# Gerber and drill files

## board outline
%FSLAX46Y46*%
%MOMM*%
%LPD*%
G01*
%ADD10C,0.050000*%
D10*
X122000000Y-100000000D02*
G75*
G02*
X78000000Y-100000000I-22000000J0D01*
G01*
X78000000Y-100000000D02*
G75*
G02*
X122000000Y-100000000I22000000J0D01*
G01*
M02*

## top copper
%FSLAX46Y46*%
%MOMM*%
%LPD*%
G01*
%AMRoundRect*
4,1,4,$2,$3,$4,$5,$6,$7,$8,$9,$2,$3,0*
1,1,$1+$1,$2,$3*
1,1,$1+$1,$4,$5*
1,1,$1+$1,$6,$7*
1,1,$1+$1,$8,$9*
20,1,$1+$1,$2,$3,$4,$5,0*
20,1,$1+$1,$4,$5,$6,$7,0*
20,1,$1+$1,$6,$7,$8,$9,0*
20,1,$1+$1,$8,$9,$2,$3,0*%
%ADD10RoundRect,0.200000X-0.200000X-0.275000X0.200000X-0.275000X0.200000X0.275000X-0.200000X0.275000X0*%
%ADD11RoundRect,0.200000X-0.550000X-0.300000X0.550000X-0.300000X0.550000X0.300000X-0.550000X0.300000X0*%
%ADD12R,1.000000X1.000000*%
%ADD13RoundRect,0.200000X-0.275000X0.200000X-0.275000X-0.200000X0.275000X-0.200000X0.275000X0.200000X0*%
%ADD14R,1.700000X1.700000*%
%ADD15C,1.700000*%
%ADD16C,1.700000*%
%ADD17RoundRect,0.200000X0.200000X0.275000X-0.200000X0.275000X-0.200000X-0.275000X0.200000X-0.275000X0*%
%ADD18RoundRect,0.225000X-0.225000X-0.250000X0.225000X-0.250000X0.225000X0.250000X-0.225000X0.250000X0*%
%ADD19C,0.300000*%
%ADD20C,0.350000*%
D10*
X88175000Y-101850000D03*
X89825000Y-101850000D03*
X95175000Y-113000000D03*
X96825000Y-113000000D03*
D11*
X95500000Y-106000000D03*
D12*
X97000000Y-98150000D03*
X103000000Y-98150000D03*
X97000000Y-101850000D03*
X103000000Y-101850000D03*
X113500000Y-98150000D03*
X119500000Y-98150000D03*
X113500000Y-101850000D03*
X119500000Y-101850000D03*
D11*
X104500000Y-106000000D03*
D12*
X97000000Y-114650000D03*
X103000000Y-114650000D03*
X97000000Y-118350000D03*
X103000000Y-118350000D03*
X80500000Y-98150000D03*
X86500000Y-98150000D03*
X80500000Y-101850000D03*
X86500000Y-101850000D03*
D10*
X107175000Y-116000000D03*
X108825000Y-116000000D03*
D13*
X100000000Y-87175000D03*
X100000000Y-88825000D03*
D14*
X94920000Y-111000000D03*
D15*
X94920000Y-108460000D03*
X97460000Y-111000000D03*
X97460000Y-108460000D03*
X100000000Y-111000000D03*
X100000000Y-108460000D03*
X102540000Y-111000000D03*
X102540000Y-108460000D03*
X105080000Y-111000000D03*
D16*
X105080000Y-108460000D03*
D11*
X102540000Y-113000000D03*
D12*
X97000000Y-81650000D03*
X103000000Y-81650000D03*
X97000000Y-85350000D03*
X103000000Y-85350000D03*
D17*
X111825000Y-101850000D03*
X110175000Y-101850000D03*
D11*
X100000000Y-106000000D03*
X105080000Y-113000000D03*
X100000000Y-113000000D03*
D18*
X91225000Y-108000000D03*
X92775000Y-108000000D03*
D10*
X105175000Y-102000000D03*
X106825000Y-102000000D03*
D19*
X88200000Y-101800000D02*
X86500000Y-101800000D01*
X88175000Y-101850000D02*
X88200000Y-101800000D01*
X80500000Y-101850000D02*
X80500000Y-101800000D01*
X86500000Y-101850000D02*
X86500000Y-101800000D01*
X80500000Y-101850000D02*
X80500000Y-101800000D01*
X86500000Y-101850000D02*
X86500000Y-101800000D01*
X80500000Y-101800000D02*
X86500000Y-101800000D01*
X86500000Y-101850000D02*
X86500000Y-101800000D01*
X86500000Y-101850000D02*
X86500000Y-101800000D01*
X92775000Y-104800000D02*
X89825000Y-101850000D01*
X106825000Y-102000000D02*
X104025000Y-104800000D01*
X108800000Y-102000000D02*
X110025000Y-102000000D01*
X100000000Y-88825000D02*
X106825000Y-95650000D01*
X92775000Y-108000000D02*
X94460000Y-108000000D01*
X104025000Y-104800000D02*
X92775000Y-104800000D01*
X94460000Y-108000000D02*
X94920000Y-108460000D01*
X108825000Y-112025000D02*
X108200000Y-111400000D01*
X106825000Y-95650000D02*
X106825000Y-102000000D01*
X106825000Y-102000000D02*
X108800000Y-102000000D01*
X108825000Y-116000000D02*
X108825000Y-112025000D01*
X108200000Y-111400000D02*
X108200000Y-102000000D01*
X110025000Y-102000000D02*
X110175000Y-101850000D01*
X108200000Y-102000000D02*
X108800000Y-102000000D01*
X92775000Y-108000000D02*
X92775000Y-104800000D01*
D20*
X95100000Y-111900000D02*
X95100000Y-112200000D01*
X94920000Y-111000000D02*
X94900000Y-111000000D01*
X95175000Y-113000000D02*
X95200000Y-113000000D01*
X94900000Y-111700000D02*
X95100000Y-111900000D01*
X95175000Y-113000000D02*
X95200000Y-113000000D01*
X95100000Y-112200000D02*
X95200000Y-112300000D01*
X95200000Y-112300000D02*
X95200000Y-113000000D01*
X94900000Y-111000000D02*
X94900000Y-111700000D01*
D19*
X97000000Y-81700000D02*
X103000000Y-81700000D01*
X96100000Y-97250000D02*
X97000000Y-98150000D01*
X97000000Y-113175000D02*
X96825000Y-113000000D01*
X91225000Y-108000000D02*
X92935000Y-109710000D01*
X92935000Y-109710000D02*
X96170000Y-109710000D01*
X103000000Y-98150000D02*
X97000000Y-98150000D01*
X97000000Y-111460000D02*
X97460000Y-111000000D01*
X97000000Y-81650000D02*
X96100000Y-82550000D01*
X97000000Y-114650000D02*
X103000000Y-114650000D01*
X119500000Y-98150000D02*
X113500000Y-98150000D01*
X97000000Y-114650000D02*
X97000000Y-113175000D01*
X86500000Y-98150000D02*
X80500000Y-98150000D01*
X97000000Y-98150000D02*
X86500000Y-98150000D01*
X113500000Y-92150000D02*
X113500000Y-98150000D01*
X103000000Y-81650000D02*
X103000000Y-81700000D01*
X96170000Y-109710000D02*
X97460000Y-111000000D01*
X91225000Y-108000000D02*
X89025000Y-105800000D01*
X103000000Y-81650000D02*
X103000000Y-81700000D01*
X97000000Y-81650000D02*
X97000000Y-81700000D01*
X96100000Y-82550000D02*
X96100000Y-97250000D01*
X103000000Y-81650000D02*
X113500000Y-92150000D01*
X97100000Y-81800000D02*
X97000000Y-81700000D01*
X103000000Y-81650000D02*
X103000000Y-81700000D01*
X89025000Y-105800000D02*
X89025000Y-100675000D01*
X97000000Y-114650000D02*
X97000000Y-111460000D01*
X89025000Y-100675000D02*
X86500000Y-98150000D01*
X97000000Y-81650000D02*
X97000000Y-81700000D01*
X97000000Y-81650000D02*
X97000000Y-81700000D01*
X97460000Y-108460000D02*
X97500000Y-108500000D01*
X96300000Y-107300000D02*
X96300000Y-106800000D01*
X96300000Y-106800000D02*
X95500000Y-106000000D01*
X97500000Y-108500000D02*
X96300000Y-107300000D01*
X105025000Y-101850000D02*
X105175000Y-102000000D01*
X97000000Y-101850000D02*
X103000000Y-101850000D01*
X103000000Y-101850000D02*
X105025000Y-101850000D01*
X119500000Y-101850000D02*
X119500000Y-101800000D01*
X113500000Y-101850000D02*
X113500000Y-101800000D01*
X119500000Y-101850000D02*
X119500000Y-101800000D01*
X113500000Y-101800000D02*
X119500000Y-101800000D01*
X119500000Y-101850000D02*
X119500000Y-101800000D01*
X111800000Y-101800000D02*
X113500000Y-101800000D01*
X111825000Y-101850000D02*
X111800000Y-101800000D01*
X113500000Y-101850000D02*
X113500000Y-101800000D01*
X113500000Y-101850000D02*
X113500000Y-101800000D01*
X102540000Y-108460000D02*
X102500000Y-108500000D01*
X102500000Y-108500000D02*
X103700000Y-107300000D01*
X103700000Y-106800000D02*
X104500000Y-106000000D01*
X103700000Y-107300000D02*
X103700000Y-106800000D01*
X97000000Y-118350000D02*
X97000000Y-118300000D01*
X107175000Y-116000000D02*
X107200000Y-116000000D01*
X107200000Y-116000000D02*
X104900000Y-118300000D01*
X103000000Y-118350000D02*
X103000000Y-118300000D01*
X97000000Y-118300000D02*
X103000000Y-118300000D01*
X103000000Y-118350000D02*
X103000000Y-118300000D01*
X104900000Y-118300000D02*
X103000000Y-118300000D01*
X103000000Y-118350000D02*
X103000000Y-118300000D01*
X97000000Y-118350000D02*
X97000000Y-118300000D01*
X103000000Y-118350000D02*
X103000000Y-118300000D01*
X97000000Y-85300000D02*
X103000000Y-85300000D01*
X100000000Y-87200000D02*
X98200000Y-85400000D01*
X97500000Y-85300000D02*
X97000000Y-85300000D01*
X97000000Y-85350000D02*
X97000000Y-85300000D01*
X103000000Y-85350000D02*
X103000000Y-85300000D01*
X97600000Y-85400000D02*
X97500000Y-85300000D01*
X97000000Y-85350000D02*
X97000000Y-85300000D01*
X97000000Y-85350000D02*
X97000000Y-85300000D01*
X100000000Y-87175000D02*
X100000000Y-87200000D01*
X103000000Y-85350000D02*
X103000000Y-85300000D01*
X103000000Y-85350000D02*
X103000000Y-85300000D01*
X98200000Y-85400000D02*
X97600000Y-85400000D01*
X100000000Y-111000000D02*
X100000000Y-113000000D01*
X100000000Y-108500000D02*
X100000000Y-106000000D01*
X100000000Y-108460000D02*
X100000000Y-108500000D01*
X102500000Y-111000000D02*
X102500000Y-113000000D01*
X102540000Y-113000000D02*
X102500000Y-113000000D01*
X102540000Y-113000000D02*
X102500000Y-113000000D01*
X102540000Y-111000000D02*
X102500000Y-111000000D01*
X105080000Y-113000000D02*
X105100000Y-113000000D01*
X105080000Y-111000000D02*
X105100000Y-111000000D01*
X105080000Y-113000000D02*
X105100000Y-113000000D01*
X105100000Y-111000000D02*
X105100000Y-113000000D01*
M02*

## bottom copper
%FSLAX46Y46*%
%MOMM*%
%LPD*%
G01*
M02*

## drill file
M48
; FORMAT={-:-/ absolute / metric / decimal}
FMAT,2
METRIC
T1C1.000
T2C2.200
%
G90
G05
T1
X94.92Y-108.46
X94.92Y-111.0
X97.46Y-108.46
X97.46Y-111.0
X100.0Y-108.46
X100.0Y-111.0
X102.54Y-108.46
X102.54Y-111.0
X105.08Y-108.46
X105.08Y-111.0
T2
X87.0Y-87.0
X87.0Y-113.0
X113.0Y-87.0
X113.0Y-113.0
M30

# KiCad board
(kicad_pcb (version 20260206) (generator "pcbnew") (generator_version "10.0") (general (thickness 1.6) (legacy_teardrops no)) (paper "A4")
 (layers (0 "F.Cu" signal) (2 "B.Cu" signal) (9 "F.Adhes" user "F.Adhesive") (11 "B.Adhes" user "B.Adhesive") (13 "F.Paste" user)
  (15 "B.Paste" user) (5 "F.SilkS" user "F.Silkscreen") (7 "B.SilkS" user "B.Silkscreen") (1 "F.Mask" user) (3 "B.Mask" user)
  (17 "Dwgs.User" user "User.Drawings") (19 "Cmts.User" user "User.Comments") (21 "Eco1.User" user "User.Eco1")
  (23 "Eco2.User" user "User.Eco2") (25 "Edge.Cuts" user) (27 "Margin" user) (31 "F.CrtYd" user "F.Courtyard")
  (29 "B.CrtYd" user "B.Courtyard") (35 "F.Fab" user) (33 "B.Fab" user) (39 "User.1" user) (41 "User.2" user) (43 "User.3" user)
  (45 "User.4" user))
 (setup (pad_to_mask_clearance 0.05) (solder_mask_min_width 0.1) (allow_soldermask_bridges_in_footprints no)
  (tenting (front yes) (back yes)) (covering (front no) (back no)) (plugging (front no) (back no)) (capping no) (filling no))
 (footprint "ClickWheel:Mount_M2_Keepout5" (layer "F.Cu") (at 87 113)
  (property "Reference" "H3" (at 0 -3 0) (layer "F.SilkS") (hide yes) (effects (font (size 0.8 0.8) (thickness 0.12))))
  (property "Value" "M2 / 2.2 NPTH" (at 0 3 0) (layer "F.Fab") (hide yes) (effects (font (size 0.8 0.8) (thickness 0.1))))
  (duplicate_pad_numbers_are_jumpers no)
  (pad "" np_thru_hole circle (at 0 0) (size 2.2 2.2) (drill 2.2) (layers "*.Cu" "*.Mask")))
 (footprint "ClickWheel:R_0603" (layer "F.Cu") (at 89 101.85)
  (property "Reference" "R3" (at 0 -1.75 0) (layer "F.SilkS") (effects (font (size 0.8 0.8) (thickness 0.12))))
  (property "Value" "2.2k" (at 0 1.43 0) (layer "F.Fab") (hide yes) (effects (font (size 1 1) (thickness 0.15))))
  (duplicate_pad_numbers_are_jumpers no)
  (pad "1" smd roundrect (at -0.825 0) (size 0.8 0.95) (layers "F.Cu" "F.Mask" "F.Paste") (roundrect_rratio 0.25) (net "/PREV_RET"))
  (pad "2" smd roundrect (at 0.825 0) (size 0.8 0.95) (layers "F.Cu" "F.Mask" "F.Paste") (roundrect_rratio 0.25) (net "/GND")))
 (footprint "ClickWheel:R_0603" (layer "F.Cu") (at 96 113)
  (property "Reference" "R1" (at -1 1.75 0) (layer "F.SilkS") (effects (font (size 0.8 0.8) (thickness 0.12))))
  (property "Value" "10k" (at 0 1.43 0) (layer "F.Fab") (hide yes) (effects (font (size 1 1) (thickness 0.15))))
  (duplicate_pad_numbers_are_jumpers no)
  (pad "1" smd roundrect (at -0.825 0) (size 0.8 0.95) (layers "F.Cu" "F.Mask" "F.Paste") (roundrect_rratio 0.25) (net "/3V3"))
  (pad "2" smd roundrect (at 0.825 0) (size 0.8 0.95) (layers "F.Cu" "F.Mask" "F.Paste") (roundrect_rratio 0.25) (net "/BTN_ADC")))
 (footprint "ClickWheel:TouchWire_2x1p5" (layer "F.Cu") (at 95.5 106)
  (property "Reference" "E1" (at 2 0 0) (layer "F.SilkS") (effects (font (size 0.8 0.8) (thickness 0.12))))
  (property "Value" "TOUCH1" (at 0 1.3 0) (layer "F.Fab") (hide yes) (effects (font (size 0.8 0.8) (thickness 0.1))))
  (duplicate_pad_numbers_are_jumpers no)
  (pad "1" smd roundrect (at 0 0) (size 1.5 1) (layers "F.Cu" "F.Mask") (roundrect_rratio 0.2) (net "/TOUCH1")))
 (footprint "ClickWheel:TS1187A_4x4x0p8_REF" (layer "F.Cu") (at 100 100)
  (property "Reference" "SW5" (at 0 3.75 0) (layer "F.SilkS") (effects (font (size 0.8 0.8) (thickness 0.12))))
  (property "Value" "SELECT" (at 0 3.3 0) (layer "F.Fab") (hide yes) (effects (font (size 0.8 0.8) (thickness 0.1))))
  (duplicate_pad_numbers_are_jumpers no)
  (pad "1" smd rect (at -3 -1.85) (size 1 1) (layers "F.Cu" "F.Mask" "F.Paste") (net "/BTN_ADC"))
  (pad "1" smd rect (at 3 -1.85) (size 1 1) (layers "F.Cu" "F.Mask" "F.Paste") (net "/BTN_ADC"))
  (pad "2" smd rect (at -3 1.85) (size 1 1) (layers "F.Cu" "F.Mask" "F.Paste") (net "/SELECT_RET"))
  (pad "2" smd rect (at 3 1.85) (size 1 1) (layers "F.Cu" "F.Mask" "F.Paste") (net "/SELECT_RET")))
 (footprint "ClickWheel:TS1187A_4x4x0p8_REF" (layer "F.Cu") (at 116.5 100)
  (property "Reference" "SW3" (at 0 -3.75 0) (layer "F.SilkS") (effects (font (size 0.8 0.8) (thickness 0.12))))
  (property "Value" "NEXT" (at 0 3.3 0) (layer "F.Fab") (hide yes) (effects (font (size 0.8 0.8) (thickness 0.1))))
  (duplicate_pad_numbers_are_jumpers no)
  (pad "1" smd rect (at -3 -1.85) (size 1 1) (layers "F.Cu" "F.Mask" "F.Paste") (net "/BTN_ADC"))
  (pad "1" smd rect (at 3 -1.85) (size 1 1) (layers "F.Cu" "F.Mask" "F.Paste") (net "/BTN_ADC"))
  (pad "2" smd rect (at -3 1.85) (size 1 1) (layers "F.Cu" "F.Mask" "F.Paste") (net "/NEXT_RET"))
  (pad "2" smd rect (at 3 1.85) (size 1 1) (layers "F.Cu" "F.Mask" "F.Paste") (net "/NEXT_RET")))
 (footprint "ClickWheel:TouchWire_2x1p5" (layer "F.Cu") (at 104.5 106)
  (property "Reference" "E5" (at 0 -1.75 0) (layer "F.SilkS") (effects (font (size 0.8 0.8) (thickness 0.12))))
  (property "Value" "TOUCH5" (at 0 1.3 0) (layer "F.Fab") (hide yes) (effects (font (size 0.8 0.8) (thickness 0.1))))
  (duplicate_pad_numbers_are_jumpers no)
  (pad "1" smd roundrect (at 0 0) (size 1.5 1) (layers "F.Cu" "F.Mask") (roundrect_rratio 0.2) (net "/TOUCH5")))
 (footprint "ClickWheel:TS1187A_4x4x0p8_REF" (layer "F.Cu") (at 100 116.5)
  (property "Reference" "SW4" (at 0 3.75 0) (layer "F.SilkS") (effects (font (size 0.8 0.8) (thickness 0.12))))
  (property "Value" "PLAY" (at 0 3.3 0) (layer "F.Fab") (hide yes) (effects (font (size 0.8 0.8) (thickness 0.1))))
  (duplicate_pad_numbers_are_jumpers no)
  (pad "1" smd rect (at -3 -1.85) (size 1 1) (layers "F.Cu" "F.Mask" "F.Paste") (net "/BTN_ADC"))
  (pad "1" smd rect (at 3 -1.85) (size 1 1) (layers "F.Cu" "F.Mask" "F.Paste") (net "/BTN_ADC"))
  (pad "2" smd rect (at -3 1.85) (size 1 1) (layers "F.Cu" "F.Mask" "F.Paste") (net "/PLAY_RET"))
  (pad "2" smd rect (at 3 1.85) (size 1 1) (layers "F.Cu" "F.Mask" "F.Paste") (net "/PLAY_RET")))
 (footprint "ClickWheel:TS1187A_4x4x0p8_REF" (layer "F.Cu") (at 83.5 100)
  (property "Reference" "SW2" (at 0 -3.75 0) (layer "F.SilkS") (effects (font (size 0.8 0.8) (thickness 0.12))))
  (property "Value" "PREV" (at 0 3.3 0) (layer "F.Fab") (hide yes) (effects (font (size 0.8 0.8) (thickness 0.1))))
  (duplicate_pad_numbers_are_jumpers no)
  (pad "1" smd rect (at -3 -1.85) (size 1 1) (layers "F.Cu" "F.Mask" "F.Paste") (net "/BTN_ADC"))
  (pad "1" smd rect (at 3 -1.85) (size 1 1) (layers "F.Cu" "F.Mask" "F.Paste") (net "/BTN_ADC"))
  (pad "2" smd rect (at -3 1.85) (size 1 1) (layers "F.Cu" "F.Mask" "F.Paste") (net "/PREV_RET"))
  (pad "2" smd rect (at 3 1.85) (size 1 1) (layers "F.Cu" "F.Mask" "F.Paste") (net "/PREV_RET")))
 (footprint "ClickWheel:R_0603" (layer "F.Cu") (at 108 116)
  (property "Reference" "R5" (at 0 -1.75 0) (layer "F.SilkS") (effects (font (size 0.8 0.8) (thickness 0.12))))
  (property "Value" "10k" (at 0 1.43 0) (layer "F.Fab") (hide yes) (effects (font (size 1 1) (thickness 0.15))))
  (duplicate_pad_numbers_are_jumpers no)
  (pad "1" smd roundrect (at -0.825 0) (size 0.8 0.95) (layers "F.Cu" "F.Mask" "F.Paste") (roundrect_rratio 0.25) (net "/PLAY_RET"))
  (pad "2" smd roundrect (at 0.825 0) (size 0.8 0.95) (layers "F.Cu" "F.Mask" "F.Paste") (roundrect_rratio 0.25) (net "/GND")))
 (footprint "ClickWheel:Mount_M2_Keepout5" (layer "F.Cu") (at 113 113)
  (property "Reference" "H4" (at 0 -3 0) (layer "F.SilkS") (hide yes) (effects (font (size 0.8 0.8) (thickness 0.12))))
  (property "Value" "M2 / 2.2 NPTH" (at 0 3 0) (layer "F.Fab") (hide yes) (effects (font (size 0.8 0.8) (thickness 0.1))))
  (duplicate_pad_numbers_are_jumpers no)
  (pad "" np_thru_hole circle (at 0 0) (size 2.2 2.2) (drill 2.2) (layers "*.Cu" "*.Mask")))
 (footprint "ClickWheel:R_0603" (layer "F.Cu") (at 100 88 -90)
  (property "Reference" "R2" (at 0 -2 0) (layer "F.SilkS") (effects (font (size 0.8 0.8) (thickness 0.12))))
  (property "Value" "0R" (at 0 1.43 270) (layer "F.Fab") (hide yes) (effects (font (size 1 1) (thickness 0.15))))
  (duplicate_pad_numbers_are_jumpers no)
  (pad "1" smd roundrect (at -0.825 0 270) (size 0.8 0.95) (layers "F.Cu" "F.Mask" "F.Paste") (roundrect_rratio 0.25) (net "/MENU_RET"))
  (pad "2" smd roundrect (at 0.825 0 270) (size 0.8 0.95) (layers "F.Cu" "F.Mask" "F.Paste") (roundrect_rratio 0.25) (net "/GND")))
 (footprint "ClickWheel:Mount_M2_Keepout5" (layer "F.Cu") (at 113 87)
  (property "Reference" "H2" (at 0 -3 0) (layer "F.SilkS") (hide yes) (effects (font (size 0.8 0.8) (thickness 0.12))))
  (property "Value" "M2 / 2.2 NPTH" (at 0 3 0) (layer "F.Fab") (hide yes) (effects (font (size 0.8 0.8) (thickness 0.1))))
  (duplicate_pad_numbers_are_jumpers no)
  (pad "" np_thru_hole circle (at 0 0) (size 2.2 2.2) (drill 2.2) (layers "*.Cu" "*.Mask")))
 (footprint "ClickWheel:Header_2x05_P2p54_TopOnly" (layer "F.Cu") (at 94.92 111 90)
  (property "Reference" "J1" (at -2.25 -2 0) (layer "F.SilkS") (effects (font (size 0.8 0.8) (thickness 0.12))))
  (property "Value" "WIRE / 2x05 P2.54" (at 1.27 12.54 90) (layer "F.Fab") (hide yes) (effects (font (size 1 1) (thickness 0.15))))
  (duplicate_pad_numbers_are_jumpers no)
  (pad "1" thru_hole rect (at 0 0 90) (size 1.7 1.7) (drill 1) (layers "*.Cu" "*.Mask") (remove_unused_layers yes) (keep_end_layers no)
   (zone_layer_connections) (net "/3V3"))
  (pad "2" thru_hole circle (at 2.54 0 90) (size 1.7 1.7) (drill 1) (layers "*.Cu" "*.Mask") (remove_unused_layers yes) (keep_end_layers no)
   (zone_layer_connections) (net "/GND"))
  (pad "3" thru_hole circle (at 0 2.54 90) (size 1.7 1.7) (drill 1) (layers "*.Cu" "*.Mask") (remove_unused_layers yes) (keep_end_layers no)
   (zone_layer_connections) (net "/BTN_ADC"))
  (pad "4" thru_hole circle (at 2.54 2.54 90) (size 1.7 1.7) (drill 1) (layers "*.Cu" "*.Mask") (remove_unused_layers yes)
   (keep_end_layers no) (zone_layer_connections) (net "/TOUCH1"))
  (pad "5" thru_hole circle (at 0 5.08 90) (size 1.7 1.7) (drill 1) (layers "*.Cu" "*.Mask") (remove_unused_layers yes) (keep_end_layers no)
   (zone_layer_connections) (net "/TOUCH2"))
  (pad "6" thru_hole circle (at 2.54 5.08 90) (size 1.7 1.7) (drill 1) (layers "*.Cu" "*.Mask") (remove_unused_layers yes)
   (keep_end_layers no) (zone_layer_connections) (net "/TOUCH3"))
  (pad "7" thru_hole circle (at 0 7.62 90) (size 1.7 1.7) (drill 1) (layers "*.Cu" "*.Mask") (remove_unused_layers yes) (keep_end_layers no)
   (zone_layer_connections) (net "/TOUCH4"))
  (pad "8" thru_hole circle (at 2.54 7.62 90) (size 1.7 1.7) (drill 1) (layers "*.Cu" "*.Mask") (remove_unused_layers yes)
   (keep_end_layers no) (zone_layer_connections) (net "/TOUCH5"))
  (pad "9" thru_hole circle (at 0 10.16 90) (size 1.7 1.7) (drill 1) (layers "*.Cu" "*.Mask") (remove_unused_layers yes)
   (keep_end_layers no) (zone_layer_connections) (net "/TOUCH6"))
  (pad "10" smd circle (at 2.54 10.16 90) (size 1.7 1.7) (layers "F.Cu" "F.Mask"))
  (pad "10" thru_hole circle (at 2.54 10.16 90) (size 1.7 1.7) (drill 1) (layers "*.Cu" "*.Mask") (remove_unused_layers yes)
   (keep_end_layers no) (zone_layer_connections)))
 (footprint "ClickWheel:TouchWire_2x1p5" (layer "F.Cu") (at 102.54 113)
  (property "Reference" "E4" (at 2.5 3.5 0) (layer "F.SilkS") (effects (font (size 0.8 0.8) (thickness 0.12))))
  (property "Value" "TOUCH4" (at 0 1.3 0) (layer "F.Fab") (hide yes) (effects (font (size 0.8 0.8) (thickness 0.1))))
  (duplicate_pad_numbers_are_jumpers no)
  (pad "1" smd roundrect (at 0 0) (size 1.5 1) (layers "F.Cu" "F.Mask") (roundrect_rratio 0.2) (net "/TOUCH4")))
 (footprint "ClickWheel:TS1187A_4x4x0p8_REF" (layer "F.Cu") (at 100 83.5)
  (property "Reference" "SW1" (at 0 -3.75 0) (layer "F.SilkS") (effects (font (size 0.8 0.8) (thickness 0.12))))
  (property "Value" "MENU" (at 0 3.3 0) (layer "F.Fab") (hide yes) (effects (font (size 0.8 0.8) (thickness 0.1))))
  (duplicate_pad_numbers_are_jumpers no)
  (pad "1" smd rect (at -3 -1.85) (size 1 1) (layers "F.Cu" "F.Mask" "F.Paste") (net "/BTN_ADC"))
  (pad "1" smd rect (at 3 -1.85) (size 1 1) (layers "F.Cu" "F.Mask" "F.Paste") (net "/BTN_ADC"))
  (pad "2" smd rect (at -3 1.85) (size 1 1) (layers "F.Cu" "F.Mask" "F.Paste") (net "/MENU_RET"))
  (pad "2" smd rect (at 3 1.85) (size 1 1) (layers "F.Cu" "F.Mask" "F.Paste") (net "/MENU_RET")))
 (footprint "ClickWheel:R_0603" (layer "F.Cu") (at 111 101.85 180)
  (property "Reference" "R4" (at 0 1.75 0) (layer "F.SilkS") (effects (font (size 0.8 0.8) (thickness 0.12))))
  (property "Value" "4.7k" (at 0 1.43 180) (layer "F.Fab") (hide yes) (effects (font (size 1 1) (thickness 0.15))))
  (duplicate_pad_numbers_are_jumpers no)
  (pad "1" smd roundrect (at -0.825 0 180) (size 0.8 0.95) (layers "F.Cu" "F.Mask" "F.Paste") (roundrect_rratio 0.25) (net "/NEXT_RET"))
  (pad "2" smd roundrect (at 0.825 0 180) (size 0.8 0.95) (layers "F.Cu" "F.Mask" "F.Paste") (roundrect_rratio 0.25) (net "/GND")))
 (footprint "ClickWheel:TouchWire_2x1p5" (layer "F.Cu") (at 100 106)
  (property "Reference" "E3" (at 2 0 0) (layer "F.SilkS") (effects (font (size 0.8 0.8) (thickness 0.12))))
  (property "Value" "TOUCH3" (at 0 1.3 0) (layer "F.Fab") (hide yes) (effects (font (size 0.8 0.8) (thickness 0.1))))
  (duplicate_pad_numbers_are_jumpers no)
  (pad "1" smd roundrect (at 0 0) (size 1.5 1) (layers "F.Cu" "F.Mask") (roundrect_rratio 0.2) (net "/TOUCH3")))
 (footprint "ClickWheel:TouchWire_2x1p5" (layer "F.Cu") (at 105.08 113)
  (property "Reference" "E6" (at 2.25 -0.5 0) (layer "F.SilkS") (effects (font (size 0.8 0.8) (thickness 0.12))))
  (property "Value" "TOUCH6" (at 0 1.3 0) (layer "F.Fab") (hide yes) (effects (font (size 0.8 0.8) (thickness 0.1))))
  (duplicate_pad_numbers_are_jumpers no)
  (pad "1" smd roundrect (at 0 0) (size 1.5 1) (layers "F.Cu" "F.Mask") (roundrect_rratio 0.2) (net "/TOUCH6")))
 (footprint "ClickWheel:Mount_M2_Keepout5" (layer "F.Cu") (at 87 87)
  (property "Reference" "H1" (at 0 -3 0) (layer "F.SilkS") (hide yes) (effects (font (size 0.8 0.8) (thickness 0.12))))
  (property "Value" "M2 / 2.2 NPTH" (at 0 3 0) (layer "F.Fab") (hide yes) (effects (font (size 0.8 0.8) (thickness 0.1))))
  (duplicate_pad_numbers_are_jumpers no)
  (pad "" np_thru_hole circle (at 0 0) (size 2.2 2.2) (drill 2.2) (layers "*.Cu" "*.Mask")))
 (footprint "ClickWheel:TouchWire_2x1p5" (layer "F.Cu") (at 100 113)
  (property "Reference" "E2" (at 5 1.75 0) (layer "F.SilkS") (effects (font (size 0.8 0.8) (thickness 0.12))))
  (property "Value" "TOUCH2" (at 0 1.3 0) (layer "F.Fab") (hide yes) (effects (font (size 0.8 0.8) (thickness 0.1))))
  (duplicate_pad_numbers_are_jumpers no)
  (pad "1" smd roundrect (at 0 0) (size 1.5 1) (layers "F.Cu" "F.Mask") (roundrect_rratio 0.2) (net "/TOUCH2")))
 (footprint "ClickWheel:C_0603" (layer "F.Cu") (at 92 108)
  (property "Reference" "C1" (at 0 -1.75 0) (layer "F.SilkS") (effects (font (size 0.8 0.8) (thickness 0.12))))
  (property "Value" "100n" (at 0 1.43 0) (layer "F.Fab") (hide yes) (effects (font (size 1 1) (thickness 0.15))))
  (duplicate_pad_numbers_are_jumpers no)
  (pad "1" smd roundrect (at -0.775 0) (size 0.9 0.95) (layers "F.Cu" "F.Mask" "F.Paste") (roundrect_rratio 0.25) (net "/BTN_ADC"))
  (pad "2" smd roundrect (at 0.775 0) (size 0.9 0.95) (layers "F.Cu" "F.Mask" "F.Paste") (roundrect_rratio 0.25) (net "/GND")))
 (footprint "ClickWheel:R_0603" (layer "F.Cu") (at 106 102)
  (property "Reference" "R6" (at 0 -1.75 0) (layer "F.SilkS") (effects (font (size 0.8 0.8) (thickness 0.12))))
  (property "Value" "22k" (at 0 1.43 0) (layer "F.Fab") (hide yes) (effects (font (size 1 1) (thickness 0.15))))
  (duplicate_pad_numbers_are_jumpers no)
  (pad "1" smd roundrect (at -0.825 0) (size 0.8 0.95) (layers "F.Cu" "F.Mask" "F.Paste") (roundrect_rratio 0.25) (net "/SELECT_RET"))
  (pad "2" smd roundrect (at 0.825 0) (size 0.8 0.95) (layers "F.Cu" "F.Mask" "F.Paste") (roundrect_rratio 0.25) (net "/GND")))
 (gr_circle (center 100 100) (end 122 100) (stroke (width 0.05) (type default)) (fill no) (layer "Edge.Cuts"))
 (segment (start 88.2 101.8) (end 86.5 101.8) (width 0.3) (layer "F.Cu") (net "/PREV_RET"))
 (segment (start 88.175 101.85) (end 88.2 101.8) (width 0.3) (layer "F.Cu") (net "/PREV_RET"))
 (segment (start 80.5 101.85) (end 80.5 101.8) (width 0.3) (layer "F.Cu") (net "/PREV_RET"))
 (segment (start 86.5 101.85) (end 86.5 101.8) (width 0.3) (layer "F.Cu") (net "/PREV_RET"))
 (segment (start 80.5 101.85) (end 80.5 101.8) (width 0.3) (layer "F.Cu") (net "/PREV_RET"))
 (segment (start 86.5 101.85) (end 86.5 101.8) (width 0.3) (layer "F.Cu") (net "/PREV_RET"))
 (segment (start 80.5 101.8) (end 86.5 101.8) (width 0.3) (layer "F.Cu") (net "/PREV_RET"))
 (segment (start 86.5 101.85) (end 86.5 101.8) (width 0.3) (layer "F.Cu") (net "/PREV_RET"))
 (segment (start 86.5 101.85) (end 86.5 101.8) (width 0.3) (layer "F.Cu") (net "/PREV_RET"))
 (segment (start 92.775 104.8) (end 89.825 101.85) (width 0.3) (layer "F.Cu") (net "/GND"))
 (segment (start 106.825 102) (end 104.025 104.8) (width 0.3) (layer "F.Cu") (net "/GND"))
 (segment (start 108.8 102) (end 110.025 102) (width 0.3) (layer "F.Cu") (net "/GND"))
 (segment (start 100 88.825) (end 106.825 95.65) (width 0.3) (layer "F.Cu") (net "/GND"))
 (segment (start 92.775 108) (end 94.46 108) (width 0.3) (layer "F.Cu") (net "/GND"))
 (segment (start 104.025 104.8) (end 92.775 104.8) (width 0.3) (layer "F.Cu") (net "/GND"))
 (segment (start 94.46 108) (end 94.92 108.46) (width 0.3) (layer "F.Cu") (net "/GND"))
 (segment (start 108.825 112.025) (end 108.2 111.4) (width 0.3) (layer "F.Cu") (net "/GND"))
 (segment (start 106.825 95.65) (end 106.825 102) (width 0.3) (layer "F.Cu") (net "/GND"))
 (segment (start 106.825 102) (end 108.8 102) (width 0.3) (layer "F.Cu") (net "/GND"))
 (segment (start 108.825 116) (end 108.825 112.025) (width 0.3) (layer "F.Cu") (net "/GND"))
 (segment (start 108.2 111.4) (end 108.2 102) (width 0.3) (layer "F.Cu") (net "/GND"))
 (segment (start 110.025 102) (end 110.175 101.85) (width 0.3) (layer "F.Cu") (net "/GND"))
 (segment (start 108.2 102) (end 108.8 102) (width 0.3) (layer "F.Cu") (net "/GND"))
 (segment (start 92.775 108) (end 92.775 104.8) (width 0.3) (layer "F.Cu") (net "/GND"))
 (segment (start 95.1 111.9) (end 95.1 112.2) (width 0.35) (layer "F.Cu") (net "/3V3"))
 (segment (start 94.92 111) (end 94.9 111) (width 0.35) (layer "F.Cu") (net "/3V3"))
 (segment (start 95.175 113) (end 95.2 113) (width 0.35) (layer "F.Cu") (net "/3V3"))
 (segment (start 94.9 111.7) (end 95.1 111.9) (width 0.35) (layer "F.Cu") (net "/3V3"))
 (segment (start 95.175 113) (end 95.2 113) (width 0.35) (layer "F.Cu") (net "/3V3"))
 (segment (start 95.1 112.2) (end 95.2 112.3) (width 0.35) (layer "F.Cu") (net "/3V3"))
 (segment (start 95.2 112.3) (end 95.2 113) (width 0.35) (layer "F.Cu") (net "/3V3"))
 (segment (start 94.9 111) (end 94.9 111.7) (width 0.35) (layer "F.Cu") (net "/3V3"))
 (segment (start 97 81.7) (end 103 81.7) (width 0.3) (layer "F.Cu") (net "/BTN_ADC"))
 (segment (start 96.1 97.25) (end 97 98.15) (width 0.3) (layer "F.Cu") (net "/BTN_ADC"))
 (segment (start 97 113.175) (end 96.825 113) (width 0.3) (layer "F.Cu") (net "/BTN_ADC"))
 (segment (start 91.225 108) (end 92.935 109.71) (width 0.3) (layer "F.Cu") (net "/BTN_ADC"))
 (segment (start 92.935 109.71) (end 96.17 109.71) (width 0.3) (layer "F.Cu") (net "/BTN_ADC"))
 (segment (start 103 98.15) (end 97 98.15) (width 0.3) (layer "F.Cu") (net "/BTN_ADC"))
 (segment (start 97 111.46) (end 97.46 111) (width 0.3) (layer "F.Cu") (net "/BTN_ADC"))
 (segment (start 97 81.65) (end 96.1 82.55) (width 0.3) (layer "F.Cu") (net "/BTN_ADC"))
 (segment (start 97 114.65) (end 103 114.65) (width 0.3) (layer "F.Cu") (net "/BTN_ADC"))
 (segment (start 119.5 98.15) (end 113.5 98.15) (width 0.3) (layer "F.Cu") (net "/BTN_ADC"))
 (segment (start 97 114.65) (end 97 113.175) (width 0.3) (layer "F.Cu") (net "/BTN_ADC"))
 (segment (start 86.5 98.15) (end 80.5 98.15) (width 0.3) (layer "F.Cu") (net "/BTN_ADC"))
 (segment (start 97 98.15) (end 86.5 98.15) (width 0.3) (layer "F.Cu") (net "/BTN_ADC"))
 (segment (start 113.5 92.15) (end 113.5 98.15) (width 0.3) (layer "F.Cu") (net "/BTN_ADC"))
 (segment (start 103 81.65) (end 103 81.7) (width 0.3) (layer "F.Cu") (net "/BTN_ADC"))
 (segment (start 96.17 109.71) (end 97.46 111) (width 0.3) (layer "F.Cu") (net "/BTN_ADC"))
 (segment (start 91.225 108) (end 89.025 105.8) (width 0.3) (layer "F.Cu") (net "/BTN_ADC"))
 (segment (start 103 81.65) (end 103 81.7) (width 0.3) (layer "F.Cu") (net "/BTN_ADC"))
 (segment (start 97 81.65) (end 97 81.7) (width 0.3) (layer "F.Cu") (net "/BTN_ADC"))
 (segment (start 96.1 82.55) (end 96.1 97.25) (width 0.3) (layer "F.Cu") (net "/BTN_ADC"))
 (segment (start 103 81.65) (end 113.5 92.15) (width 0.3) (layer "F.Cu") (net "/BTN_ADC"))
 (segment (start 97.1 81.8) (end 97 81.7) (width 0.3) (layer "F.Cu") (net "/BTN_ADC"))
 (segment (start 103 81.65) (end 103 81.7) (width 0.3) (layer "F.Cu") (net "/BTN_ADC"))
 (segment (start 89.025 105.8) (end 89.025 100.675) (width 0.3) (layer "F.Cu") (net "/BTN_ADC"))
 (segment (start 97 114.65) (end 97 111.46) (width 0.3) (layer "F.Cu") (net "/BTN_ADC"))
 (segment (start 89.025 100.675) (end 86.5 98.15) (width 0.3) (layer "F.Cu") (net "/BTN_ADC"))
 (segment (start 97 81.65) (end 97 81.7) (width 0.3) (layer "F.Cu") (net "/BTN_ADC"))
 (segment (start 97 81.65) (end 97 81.7) (width 0.3) (layer "F.Cu") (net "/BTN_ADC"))
 (segment (start 97.46 108.46) (end 97.5 108.5) (width 0.3) (layer "F.Cu") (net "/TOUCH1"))
 (segment (start 96.3 107.3) (end 96.3 106.8) (width 0.3) (layer "F.Cu") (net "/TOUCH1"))
 (segment (start 96.3 106.8) (end 95.5 106) (width 0.3) (layer "F.Cu") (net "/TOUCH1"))
 (segment (start 97.5 108.5) (end 96.3 107.3) (width 0.3) (layer "F.Cu") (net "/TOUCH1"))
 (segment (start 105.025 101.85) (end 105.175 102) (width 0.3) (layer "F.Cu") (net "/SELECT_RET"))
 (segment (start 97 101.85) (end 103 101.85) (width 0.3) (layer "F.Cu") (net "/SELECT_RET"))
 (segment (start 103 101.85) (end 105.025 101.85) (width 0.3) (layer "F.Cu") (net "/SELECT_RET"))
 (segment (start 119.5 101.85) (end 119.5 101.8) (width 0.3) (layer "F.Cu") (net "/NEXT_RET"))
 (segment (start 113.5 101.85) (end 113.5 101.8) (width 0.3) (layer "F.Cu") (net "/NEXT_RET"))
 (segment (start 119.5 101.85) (end 119.5 101.8) (width 0.3) (layer "F.Cu") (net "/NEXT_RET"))
 (segment (start 113.5 101.8) (end 119.5 101.8) (width 0.3) (layer "F.Cu") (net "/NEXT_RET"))
 (segment (start 119.5 101.85) (end 119.5 101.8) (width 0.3) (layer "F.Cu") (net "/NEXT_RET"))
 (segment (start 111.8 101.8) (end 113.5 101.8) (width 0.3) (layer "F.Cu") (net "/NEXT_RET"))
 (segment (start 111.825 101.85) (end 111.8 101.8) (width 0.3) (layer "F.Cu") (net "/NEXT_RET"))
 (segment (start 113.5 101.85) (end 113.5 101.8) (width 0.3) (layer "F.Cu") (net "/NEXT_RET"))
 (segment (start 113.5 101.85) (end 113.5 101.8) (width 0.3) (layer "F.Cu") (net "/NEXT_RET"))
 (segment (start 102.54 108.46) (end 102.5 108.5) (width 0.3) (layer "F.Cu") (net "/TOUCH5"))
 (segment (start 102.5 108.5) (end 103.7 107.3) (width 0.3) (layer "F.Cu") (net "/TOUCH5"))
 (segment (start 103.7 106.8) (end 104.5 106) (width 0.3) (layer "F.Cu") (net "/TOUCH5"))
 (segment (start 103.7 107.3) (end 103.7 106.8) (width 0.3) (layer "F.Cu") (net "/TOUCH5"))
 (segment (start 97 118.35) (end 97 118.3) (width 0.3) (layer "F.Cu") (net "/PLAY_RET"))
 (segment (start 107.175 116) (end 107.2 116) (width 0.3) (layer "F.Cu") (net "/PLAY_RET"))
 (segment (start 107.2 116) (end 104.9 118.3) (width 0.3) (layer "F.Cu") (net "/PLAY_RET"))
 (segment (start 103 118.35) (end 103 118.3) (width 0.3) (layer "F.Cu") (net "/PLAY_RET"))
 (segment (start 97 118.3) (end 103 118.3) (width 0.3) (layer "F.Cu") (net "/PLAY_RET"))
 (segment (start 103 118.35) (end 103 118.3) (width 0.3) (layer "F.Cu") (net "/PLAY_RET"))
 (segment (start 104.9 118.3) (end 103 118.3) (width 0.3) (layer "F.Cu") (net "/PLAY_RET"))
 (segment (start 103 118.35) (end 103 118.3) (width 0.3) (layer "F.Cu") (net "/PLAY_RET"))
 (segment (start 97 118.35) (end 97 118.3) (width 0.3) (layer "F.Cu") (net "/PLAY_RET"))
 (segment (start 103 118.35) (end 103 118.3) (width 0.3) (layer "F.Cu") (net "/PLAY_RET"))
 (segment (start 97 85.3) (end 103 85.3) (width 0.3) (layer "F.Cu") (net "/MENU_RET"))
 (segment (start 100 87.2) (end 98.2 85.4) (width 0.3) (layer "F.Cu") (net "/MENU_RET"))
 (segment (start 97.5 85.3) (end 97 85.3) (width 0.3) (layer "F.Cu") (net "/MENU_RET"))
 (segment (start 97 85.35) (end 97 85.3) (width 0.3) (layer "F.Cu") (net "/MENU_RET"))
 (segment (start 103 85.35) (end 103 85.3) (width 0.3) (layer "F.Cu") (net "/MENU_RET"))
 (segment (start 97.6 85.4) (end 97.5 85.3) (width 0.3) (layer "F.Cu") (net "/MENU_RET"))
 (segment (start 97 85.35) (end 97 85.3) (width 0.3) (layer "F.Cu") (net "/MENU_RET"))
 (segment (start 97 85.35) (end 97 85.3) (width 0.3) (layer "F.Cu") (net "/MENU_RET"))
 (segment (start 100 87.175) (end 100 87.2) (width 0.3) (layer "F.Cu") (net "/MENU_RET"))
 (segment (start 103 85.35) (end 103 85.3) (width 0.3) (layer "F.Cu") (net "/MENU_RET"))
 (segment (start 103 85.35) (end 103 85.3) (width 0.3) (layer "F.Cu") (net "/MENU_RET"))
 (segment (start 98.2 85.4) (end 97.6 85.4) (width 0.3) (layer "F.Cu") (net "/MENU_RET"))
 (segment (start 100 111) (end 100 113) (width 0.3) (layer "F.Cu") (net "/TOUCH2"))
 (segment (start 100 108.5) (end 100 106) (width 0.3) (layer "F.Cu") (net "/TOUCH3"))
 (segment (start 100 108.46) (end 100 108.5) (width 0.3) (layer "F.Cu") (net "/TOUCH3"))
 (segment (start 102.5 111) (end 102.5 113) (width 0.3) (layer "F.Cu") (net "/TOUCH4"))
 (segment (start 102.54 113) (end 102.5 113) (width 0.3) (layer "F.Cu") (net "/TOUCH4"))
 (segment (start 102.54 113) (end 102.5 113) (width 0.3) (layer "F.Cu") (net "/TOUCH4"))
 (segment (start 102.54 111) (end 102.5 111) (width 0.3) (layer "F.Cu") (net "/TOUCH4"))
 (segment (start 105.08 113) (end 105.1 113) (width 0.3) (layer "F.Cu") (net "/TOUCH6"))
 (segment (start 105.08 111) (end 105.1 111) (width 0.3) (layer "F.Cu") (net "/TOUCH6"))
 (segment (start 105.08 113) (end 105.1 113) (width 0.3) (layer "F.Cu") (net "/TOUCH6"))
 (segment (start 105.1 111) (end 105.1 113) (width 0.3) (layer "F.Cu") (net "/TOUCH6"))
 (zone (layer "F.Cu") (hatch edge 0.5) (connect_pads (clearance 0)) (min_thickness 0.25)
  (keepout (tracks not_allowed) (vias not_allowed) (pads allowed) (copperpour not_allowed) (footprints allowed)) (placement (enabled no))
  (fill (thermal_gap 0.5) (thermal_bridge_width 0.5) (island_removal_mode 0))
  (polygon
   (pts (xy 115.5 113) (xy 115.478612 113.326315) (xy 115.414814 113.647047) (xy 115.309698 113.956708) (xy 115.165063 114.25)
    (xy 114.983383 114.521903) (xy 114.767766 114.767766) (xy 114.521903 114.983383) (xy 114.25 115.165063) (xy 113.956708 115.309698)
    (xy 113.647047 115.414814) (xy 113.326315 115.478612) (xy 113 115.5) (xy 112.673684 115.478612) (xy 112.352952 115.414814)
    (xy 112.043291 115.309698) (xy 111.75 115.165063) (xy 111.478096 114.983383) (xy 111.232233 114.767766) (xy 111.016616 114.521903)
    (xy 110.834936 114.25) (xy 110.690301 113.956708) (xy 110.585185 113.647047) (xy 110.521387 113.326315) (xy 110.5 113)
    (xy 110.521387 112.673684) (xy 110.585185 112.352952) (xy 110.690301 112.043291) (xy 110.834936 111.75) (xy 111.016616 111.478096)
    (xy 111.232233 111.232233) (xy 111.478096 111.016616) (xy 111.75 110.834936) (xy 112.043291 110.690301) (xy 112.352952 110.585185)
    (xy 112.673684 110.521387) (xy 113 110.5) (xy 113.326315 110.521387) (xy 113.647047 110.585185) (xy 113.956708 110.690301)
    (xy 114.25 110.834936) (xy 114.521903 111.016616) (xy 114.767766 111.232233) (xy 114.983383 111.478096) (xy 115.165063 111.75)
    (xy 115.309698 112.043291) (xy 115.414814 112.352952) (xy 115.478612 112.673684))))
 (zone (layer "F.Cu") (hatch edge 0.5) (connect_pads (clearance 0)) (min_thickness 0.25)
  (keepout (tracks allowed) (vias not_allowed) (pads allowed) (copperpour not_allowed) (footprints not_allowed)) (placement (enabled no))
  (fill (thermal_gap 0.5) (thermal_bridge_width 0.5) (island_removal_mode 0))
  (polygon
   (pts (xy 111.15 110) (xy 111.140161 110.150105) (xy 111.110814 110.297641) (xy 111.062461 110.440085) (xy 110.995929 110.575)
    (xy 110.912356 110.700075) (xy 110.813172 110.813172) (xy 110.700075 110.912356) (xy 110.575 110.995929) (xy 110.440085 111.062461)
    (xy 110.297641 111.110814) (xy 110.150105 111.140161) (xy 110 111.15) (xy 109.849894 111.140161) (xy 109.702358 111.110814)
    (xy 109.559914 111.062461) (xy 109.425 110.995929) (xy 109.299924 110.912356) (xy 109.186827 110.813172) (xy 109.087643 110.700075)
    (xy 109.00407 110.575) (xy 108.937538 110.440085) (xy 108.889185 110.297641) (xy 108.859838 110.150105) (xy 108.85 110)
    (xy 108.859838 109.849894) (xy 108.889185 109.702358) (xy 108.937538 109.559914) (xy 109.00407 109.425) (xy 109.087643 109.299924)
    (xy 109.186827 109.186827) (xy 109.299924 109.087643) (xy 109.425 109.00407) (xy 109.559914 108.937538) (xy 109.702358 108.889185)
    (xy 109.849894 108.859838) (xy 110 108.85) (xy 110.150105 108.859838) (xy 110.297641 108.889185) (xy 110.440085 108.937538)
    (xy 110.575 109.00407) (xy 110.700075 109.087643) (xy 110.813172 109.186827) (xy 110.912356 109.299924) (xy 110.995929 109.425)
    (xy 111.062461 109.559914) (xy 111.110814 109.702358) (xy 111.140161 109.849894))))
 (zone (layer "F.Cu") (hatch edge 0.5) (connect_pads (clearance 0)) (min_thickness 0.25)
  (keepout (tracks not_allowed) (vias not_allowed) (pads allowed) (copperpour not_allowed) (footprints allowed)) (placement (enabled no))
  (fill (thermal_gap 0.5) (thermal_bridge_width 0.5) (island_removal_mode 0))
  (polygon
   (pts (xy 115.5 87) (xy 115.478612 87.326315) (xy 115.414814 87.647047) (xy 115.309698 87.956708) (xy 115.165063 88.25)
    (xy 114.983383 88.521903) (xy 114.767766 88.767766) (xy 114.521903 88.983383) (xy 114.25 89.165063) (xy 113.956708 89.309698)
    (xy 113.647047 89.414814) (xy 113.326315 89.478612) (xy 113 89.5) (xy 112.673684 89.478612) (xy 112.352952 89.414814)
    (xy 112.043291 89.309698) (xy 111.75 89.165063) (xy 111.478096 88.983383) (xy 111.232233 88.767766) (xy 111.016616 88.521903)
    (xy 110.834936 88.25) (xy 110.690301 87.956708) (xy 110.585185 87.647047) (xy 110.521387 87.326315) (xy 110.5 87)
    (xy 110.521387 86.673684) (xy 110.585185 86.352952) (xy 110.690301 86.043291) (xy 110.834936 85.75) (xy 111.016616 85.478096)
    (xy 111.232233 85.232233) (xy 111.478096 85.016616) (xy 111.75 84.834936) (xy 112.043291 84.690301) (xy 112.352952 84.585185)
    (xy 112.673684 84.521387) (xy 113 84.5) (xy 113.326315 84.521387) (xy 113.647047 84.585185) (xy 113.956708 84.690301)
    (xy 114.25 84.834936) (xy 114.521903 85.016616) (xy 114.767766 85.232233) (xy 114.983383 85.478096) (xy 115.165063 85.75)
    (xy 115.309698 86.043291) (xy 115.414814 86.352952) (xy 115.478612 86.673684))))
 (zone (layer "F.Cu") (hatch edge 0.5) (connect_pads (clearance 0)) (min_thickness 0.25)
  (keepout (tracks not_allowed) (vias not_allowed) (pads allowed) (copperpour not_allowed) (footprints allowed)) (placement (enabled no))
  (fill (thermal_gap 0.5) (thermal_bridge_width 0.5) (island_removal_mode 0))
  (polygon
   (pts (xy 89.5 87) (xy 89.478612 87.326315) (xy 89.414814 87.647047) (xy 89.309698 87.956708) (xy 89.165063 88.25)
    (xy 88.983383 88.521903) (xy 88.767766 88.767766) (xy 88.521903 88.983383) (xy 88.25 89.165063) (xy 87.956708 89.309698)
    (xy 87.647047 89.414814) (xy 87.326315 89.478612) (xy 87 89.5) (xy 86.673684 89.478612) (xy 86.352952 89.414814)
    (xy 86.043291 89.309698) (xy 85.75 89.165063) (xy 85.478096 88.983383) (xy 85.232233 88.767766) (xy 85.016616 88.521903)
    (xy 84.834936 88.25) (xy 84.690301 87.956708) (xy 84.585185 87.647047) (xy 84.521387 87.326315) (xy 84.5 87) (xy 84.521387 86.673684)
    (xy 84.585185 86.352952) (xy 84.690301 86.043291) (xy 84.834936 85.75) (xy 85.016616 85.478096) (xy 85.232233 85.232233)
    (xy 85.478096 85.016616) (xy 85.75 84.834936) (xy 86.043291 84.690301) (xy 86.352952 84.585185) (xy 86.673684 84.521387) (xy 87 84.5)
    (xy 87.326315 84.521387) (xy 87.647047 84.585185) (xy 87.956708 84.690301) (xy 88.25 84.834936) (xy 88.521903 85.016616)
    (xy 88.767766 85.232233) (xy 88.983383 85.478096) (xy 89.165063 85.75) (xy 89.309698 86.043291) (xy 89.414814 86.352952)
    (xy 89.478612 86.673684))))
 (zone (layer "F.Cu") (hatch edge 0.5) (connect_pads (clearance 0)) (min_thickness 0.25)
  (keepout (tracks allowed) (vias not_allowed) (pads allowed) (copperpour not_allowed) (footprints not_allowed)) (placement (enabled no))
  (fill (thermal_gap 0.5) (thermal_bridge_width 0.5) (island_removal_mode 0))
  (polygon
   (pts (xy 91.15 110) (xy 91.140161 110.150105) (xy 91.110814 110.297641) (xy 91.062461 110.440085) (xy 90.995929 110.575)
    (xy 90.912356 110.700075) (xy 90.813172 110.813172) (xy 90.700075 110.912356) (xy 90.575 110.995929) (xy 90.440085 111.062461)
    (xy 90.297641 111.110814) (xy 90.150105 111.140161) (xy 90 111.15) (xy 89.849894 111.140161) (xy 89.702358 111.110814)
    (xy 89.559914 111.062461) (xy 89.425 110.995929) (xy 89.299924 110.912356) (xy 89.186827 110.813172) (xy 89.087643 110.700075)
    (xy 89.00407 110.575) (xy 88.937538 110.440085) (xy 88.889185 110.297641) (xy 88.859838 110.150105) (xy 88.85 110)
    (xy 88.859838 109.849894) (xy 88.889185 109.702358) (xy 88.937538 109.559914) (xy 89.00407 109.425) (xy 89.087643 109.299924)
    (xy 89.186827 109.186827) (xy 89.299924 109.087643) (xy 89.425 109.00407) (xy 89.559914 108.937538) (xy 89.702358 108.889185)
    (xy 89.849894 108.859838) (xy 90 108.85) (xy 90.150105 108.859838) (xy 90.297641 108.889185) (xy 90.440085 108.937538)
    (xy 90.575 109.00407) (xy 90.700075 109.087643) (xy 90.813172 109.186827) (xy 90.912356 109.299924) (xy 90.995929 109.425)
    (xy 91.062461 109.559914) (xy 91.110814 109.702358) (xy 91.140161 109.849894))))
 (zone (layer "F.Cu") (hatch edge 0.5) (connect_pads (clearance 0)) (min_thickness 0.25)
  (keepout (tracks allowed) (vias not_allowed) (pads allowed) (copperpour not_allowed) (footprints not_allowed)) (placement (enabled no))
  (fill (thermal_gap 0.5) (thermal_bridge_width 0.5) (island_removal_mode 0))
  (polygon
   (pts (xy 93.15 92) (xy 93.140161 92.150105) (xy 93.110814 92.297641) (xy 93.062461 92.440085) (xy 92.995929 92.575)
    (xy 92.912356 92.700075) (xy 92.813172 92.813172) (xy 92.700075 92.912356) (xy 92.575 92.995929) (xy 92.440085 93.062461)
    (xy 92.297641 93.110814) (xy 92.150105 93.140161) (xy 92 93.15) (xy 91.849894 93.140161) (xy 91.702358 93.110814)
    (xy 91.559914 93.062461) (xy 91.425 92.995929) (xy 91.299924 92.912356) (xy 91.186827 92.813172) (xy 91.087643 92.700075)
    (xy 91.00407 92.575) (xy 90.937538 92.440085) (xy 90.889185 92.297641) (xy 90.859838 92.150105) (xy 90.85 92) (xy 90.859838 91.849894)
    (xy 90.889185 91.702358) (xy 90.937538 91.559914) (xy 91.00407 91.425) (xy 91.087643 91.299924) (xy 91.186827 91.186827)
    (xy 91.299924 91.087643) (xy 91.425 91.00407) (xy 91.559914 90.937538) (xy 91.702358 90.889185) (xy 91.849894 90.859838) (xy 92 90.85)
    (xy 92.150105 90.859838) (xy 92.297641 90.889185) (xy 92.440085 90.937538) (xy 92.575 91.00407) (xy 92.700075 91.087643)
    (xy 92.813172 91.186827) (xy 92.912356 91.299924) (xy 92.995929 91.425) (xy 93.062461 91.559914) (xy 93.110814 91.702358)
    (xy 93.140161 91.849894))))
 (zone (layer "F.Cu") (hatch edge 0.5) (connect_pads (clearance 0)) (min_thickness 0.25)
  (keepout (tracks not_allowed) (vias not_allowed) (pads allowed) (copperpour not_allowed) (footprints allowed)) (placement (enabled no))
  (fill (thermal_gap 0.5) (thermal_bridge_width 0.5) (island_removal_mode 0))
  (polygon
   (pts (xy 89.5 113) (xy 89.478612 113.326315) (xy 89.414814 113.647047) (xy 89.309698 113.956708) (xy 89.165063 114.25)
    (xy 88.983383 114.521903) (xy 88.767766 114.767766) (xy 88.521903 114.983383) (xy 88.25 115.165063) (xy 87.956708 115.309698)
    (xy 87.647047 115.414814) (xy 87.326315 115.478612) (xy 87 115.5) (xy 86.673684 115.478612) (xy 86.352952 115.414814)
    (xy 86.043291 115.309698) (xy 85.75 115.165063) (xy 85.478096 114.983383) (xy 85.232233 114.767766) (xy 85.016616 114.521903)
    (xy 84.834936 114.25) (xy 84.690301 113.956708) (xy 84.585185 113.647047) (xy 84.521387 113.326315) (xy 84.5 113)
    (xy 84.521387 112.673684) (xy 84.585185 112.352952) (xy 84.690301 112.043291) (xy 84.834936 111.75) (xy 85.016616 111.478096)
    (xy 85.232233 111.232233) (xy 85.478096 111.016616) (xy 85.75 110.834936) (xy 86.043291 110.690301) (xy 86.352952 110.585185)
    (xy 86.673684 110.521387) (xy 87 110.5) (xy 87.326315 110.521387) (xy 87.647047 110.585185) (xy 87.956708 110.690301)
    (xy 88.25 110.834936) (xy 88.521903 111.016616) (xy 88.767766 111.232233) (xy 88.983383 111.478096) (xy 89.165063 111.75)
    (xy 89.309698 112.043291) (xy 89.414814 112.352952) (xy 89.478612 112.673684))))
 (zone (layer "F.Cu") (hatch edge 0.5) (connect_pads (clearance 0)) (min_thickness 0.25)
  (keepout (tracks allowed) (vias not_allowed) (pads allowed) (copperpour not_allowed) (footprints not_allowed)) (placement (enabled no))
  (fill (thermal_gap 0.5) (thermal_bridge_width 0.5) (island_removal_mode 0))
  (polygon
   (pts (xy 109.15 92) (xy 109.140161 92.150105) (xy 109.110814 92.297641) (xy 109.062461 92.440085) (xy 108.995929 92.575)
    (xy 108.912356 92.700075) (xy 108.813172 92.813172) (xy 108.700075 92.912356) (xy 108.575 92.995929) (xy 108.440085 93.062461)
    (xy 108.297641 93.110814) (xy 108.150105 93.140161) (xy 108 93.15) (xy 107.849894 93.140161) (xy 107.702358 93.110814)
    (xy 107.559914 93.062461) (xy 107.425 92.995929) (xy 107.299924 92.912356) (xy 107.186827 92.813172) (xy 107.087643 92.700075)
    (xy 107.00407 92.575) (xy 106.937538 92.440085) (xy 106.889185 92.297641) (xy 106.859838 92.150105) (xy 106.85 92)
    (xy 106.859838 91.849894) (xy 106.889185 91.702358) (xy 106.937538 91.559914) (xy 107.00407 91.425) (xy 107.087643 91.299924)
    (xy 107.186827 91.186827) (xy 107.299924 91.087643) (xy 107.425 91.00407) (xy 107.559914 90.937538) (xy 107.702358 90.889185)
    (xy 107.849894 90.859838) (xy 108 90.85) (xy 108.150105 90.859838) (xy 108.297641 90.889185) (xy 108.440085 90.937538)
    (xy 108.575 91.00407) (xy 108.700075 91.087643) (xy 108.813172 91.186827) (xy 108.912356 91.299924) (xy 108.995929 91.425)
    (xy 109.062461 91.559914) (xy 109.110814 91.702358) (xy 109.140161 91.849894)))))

